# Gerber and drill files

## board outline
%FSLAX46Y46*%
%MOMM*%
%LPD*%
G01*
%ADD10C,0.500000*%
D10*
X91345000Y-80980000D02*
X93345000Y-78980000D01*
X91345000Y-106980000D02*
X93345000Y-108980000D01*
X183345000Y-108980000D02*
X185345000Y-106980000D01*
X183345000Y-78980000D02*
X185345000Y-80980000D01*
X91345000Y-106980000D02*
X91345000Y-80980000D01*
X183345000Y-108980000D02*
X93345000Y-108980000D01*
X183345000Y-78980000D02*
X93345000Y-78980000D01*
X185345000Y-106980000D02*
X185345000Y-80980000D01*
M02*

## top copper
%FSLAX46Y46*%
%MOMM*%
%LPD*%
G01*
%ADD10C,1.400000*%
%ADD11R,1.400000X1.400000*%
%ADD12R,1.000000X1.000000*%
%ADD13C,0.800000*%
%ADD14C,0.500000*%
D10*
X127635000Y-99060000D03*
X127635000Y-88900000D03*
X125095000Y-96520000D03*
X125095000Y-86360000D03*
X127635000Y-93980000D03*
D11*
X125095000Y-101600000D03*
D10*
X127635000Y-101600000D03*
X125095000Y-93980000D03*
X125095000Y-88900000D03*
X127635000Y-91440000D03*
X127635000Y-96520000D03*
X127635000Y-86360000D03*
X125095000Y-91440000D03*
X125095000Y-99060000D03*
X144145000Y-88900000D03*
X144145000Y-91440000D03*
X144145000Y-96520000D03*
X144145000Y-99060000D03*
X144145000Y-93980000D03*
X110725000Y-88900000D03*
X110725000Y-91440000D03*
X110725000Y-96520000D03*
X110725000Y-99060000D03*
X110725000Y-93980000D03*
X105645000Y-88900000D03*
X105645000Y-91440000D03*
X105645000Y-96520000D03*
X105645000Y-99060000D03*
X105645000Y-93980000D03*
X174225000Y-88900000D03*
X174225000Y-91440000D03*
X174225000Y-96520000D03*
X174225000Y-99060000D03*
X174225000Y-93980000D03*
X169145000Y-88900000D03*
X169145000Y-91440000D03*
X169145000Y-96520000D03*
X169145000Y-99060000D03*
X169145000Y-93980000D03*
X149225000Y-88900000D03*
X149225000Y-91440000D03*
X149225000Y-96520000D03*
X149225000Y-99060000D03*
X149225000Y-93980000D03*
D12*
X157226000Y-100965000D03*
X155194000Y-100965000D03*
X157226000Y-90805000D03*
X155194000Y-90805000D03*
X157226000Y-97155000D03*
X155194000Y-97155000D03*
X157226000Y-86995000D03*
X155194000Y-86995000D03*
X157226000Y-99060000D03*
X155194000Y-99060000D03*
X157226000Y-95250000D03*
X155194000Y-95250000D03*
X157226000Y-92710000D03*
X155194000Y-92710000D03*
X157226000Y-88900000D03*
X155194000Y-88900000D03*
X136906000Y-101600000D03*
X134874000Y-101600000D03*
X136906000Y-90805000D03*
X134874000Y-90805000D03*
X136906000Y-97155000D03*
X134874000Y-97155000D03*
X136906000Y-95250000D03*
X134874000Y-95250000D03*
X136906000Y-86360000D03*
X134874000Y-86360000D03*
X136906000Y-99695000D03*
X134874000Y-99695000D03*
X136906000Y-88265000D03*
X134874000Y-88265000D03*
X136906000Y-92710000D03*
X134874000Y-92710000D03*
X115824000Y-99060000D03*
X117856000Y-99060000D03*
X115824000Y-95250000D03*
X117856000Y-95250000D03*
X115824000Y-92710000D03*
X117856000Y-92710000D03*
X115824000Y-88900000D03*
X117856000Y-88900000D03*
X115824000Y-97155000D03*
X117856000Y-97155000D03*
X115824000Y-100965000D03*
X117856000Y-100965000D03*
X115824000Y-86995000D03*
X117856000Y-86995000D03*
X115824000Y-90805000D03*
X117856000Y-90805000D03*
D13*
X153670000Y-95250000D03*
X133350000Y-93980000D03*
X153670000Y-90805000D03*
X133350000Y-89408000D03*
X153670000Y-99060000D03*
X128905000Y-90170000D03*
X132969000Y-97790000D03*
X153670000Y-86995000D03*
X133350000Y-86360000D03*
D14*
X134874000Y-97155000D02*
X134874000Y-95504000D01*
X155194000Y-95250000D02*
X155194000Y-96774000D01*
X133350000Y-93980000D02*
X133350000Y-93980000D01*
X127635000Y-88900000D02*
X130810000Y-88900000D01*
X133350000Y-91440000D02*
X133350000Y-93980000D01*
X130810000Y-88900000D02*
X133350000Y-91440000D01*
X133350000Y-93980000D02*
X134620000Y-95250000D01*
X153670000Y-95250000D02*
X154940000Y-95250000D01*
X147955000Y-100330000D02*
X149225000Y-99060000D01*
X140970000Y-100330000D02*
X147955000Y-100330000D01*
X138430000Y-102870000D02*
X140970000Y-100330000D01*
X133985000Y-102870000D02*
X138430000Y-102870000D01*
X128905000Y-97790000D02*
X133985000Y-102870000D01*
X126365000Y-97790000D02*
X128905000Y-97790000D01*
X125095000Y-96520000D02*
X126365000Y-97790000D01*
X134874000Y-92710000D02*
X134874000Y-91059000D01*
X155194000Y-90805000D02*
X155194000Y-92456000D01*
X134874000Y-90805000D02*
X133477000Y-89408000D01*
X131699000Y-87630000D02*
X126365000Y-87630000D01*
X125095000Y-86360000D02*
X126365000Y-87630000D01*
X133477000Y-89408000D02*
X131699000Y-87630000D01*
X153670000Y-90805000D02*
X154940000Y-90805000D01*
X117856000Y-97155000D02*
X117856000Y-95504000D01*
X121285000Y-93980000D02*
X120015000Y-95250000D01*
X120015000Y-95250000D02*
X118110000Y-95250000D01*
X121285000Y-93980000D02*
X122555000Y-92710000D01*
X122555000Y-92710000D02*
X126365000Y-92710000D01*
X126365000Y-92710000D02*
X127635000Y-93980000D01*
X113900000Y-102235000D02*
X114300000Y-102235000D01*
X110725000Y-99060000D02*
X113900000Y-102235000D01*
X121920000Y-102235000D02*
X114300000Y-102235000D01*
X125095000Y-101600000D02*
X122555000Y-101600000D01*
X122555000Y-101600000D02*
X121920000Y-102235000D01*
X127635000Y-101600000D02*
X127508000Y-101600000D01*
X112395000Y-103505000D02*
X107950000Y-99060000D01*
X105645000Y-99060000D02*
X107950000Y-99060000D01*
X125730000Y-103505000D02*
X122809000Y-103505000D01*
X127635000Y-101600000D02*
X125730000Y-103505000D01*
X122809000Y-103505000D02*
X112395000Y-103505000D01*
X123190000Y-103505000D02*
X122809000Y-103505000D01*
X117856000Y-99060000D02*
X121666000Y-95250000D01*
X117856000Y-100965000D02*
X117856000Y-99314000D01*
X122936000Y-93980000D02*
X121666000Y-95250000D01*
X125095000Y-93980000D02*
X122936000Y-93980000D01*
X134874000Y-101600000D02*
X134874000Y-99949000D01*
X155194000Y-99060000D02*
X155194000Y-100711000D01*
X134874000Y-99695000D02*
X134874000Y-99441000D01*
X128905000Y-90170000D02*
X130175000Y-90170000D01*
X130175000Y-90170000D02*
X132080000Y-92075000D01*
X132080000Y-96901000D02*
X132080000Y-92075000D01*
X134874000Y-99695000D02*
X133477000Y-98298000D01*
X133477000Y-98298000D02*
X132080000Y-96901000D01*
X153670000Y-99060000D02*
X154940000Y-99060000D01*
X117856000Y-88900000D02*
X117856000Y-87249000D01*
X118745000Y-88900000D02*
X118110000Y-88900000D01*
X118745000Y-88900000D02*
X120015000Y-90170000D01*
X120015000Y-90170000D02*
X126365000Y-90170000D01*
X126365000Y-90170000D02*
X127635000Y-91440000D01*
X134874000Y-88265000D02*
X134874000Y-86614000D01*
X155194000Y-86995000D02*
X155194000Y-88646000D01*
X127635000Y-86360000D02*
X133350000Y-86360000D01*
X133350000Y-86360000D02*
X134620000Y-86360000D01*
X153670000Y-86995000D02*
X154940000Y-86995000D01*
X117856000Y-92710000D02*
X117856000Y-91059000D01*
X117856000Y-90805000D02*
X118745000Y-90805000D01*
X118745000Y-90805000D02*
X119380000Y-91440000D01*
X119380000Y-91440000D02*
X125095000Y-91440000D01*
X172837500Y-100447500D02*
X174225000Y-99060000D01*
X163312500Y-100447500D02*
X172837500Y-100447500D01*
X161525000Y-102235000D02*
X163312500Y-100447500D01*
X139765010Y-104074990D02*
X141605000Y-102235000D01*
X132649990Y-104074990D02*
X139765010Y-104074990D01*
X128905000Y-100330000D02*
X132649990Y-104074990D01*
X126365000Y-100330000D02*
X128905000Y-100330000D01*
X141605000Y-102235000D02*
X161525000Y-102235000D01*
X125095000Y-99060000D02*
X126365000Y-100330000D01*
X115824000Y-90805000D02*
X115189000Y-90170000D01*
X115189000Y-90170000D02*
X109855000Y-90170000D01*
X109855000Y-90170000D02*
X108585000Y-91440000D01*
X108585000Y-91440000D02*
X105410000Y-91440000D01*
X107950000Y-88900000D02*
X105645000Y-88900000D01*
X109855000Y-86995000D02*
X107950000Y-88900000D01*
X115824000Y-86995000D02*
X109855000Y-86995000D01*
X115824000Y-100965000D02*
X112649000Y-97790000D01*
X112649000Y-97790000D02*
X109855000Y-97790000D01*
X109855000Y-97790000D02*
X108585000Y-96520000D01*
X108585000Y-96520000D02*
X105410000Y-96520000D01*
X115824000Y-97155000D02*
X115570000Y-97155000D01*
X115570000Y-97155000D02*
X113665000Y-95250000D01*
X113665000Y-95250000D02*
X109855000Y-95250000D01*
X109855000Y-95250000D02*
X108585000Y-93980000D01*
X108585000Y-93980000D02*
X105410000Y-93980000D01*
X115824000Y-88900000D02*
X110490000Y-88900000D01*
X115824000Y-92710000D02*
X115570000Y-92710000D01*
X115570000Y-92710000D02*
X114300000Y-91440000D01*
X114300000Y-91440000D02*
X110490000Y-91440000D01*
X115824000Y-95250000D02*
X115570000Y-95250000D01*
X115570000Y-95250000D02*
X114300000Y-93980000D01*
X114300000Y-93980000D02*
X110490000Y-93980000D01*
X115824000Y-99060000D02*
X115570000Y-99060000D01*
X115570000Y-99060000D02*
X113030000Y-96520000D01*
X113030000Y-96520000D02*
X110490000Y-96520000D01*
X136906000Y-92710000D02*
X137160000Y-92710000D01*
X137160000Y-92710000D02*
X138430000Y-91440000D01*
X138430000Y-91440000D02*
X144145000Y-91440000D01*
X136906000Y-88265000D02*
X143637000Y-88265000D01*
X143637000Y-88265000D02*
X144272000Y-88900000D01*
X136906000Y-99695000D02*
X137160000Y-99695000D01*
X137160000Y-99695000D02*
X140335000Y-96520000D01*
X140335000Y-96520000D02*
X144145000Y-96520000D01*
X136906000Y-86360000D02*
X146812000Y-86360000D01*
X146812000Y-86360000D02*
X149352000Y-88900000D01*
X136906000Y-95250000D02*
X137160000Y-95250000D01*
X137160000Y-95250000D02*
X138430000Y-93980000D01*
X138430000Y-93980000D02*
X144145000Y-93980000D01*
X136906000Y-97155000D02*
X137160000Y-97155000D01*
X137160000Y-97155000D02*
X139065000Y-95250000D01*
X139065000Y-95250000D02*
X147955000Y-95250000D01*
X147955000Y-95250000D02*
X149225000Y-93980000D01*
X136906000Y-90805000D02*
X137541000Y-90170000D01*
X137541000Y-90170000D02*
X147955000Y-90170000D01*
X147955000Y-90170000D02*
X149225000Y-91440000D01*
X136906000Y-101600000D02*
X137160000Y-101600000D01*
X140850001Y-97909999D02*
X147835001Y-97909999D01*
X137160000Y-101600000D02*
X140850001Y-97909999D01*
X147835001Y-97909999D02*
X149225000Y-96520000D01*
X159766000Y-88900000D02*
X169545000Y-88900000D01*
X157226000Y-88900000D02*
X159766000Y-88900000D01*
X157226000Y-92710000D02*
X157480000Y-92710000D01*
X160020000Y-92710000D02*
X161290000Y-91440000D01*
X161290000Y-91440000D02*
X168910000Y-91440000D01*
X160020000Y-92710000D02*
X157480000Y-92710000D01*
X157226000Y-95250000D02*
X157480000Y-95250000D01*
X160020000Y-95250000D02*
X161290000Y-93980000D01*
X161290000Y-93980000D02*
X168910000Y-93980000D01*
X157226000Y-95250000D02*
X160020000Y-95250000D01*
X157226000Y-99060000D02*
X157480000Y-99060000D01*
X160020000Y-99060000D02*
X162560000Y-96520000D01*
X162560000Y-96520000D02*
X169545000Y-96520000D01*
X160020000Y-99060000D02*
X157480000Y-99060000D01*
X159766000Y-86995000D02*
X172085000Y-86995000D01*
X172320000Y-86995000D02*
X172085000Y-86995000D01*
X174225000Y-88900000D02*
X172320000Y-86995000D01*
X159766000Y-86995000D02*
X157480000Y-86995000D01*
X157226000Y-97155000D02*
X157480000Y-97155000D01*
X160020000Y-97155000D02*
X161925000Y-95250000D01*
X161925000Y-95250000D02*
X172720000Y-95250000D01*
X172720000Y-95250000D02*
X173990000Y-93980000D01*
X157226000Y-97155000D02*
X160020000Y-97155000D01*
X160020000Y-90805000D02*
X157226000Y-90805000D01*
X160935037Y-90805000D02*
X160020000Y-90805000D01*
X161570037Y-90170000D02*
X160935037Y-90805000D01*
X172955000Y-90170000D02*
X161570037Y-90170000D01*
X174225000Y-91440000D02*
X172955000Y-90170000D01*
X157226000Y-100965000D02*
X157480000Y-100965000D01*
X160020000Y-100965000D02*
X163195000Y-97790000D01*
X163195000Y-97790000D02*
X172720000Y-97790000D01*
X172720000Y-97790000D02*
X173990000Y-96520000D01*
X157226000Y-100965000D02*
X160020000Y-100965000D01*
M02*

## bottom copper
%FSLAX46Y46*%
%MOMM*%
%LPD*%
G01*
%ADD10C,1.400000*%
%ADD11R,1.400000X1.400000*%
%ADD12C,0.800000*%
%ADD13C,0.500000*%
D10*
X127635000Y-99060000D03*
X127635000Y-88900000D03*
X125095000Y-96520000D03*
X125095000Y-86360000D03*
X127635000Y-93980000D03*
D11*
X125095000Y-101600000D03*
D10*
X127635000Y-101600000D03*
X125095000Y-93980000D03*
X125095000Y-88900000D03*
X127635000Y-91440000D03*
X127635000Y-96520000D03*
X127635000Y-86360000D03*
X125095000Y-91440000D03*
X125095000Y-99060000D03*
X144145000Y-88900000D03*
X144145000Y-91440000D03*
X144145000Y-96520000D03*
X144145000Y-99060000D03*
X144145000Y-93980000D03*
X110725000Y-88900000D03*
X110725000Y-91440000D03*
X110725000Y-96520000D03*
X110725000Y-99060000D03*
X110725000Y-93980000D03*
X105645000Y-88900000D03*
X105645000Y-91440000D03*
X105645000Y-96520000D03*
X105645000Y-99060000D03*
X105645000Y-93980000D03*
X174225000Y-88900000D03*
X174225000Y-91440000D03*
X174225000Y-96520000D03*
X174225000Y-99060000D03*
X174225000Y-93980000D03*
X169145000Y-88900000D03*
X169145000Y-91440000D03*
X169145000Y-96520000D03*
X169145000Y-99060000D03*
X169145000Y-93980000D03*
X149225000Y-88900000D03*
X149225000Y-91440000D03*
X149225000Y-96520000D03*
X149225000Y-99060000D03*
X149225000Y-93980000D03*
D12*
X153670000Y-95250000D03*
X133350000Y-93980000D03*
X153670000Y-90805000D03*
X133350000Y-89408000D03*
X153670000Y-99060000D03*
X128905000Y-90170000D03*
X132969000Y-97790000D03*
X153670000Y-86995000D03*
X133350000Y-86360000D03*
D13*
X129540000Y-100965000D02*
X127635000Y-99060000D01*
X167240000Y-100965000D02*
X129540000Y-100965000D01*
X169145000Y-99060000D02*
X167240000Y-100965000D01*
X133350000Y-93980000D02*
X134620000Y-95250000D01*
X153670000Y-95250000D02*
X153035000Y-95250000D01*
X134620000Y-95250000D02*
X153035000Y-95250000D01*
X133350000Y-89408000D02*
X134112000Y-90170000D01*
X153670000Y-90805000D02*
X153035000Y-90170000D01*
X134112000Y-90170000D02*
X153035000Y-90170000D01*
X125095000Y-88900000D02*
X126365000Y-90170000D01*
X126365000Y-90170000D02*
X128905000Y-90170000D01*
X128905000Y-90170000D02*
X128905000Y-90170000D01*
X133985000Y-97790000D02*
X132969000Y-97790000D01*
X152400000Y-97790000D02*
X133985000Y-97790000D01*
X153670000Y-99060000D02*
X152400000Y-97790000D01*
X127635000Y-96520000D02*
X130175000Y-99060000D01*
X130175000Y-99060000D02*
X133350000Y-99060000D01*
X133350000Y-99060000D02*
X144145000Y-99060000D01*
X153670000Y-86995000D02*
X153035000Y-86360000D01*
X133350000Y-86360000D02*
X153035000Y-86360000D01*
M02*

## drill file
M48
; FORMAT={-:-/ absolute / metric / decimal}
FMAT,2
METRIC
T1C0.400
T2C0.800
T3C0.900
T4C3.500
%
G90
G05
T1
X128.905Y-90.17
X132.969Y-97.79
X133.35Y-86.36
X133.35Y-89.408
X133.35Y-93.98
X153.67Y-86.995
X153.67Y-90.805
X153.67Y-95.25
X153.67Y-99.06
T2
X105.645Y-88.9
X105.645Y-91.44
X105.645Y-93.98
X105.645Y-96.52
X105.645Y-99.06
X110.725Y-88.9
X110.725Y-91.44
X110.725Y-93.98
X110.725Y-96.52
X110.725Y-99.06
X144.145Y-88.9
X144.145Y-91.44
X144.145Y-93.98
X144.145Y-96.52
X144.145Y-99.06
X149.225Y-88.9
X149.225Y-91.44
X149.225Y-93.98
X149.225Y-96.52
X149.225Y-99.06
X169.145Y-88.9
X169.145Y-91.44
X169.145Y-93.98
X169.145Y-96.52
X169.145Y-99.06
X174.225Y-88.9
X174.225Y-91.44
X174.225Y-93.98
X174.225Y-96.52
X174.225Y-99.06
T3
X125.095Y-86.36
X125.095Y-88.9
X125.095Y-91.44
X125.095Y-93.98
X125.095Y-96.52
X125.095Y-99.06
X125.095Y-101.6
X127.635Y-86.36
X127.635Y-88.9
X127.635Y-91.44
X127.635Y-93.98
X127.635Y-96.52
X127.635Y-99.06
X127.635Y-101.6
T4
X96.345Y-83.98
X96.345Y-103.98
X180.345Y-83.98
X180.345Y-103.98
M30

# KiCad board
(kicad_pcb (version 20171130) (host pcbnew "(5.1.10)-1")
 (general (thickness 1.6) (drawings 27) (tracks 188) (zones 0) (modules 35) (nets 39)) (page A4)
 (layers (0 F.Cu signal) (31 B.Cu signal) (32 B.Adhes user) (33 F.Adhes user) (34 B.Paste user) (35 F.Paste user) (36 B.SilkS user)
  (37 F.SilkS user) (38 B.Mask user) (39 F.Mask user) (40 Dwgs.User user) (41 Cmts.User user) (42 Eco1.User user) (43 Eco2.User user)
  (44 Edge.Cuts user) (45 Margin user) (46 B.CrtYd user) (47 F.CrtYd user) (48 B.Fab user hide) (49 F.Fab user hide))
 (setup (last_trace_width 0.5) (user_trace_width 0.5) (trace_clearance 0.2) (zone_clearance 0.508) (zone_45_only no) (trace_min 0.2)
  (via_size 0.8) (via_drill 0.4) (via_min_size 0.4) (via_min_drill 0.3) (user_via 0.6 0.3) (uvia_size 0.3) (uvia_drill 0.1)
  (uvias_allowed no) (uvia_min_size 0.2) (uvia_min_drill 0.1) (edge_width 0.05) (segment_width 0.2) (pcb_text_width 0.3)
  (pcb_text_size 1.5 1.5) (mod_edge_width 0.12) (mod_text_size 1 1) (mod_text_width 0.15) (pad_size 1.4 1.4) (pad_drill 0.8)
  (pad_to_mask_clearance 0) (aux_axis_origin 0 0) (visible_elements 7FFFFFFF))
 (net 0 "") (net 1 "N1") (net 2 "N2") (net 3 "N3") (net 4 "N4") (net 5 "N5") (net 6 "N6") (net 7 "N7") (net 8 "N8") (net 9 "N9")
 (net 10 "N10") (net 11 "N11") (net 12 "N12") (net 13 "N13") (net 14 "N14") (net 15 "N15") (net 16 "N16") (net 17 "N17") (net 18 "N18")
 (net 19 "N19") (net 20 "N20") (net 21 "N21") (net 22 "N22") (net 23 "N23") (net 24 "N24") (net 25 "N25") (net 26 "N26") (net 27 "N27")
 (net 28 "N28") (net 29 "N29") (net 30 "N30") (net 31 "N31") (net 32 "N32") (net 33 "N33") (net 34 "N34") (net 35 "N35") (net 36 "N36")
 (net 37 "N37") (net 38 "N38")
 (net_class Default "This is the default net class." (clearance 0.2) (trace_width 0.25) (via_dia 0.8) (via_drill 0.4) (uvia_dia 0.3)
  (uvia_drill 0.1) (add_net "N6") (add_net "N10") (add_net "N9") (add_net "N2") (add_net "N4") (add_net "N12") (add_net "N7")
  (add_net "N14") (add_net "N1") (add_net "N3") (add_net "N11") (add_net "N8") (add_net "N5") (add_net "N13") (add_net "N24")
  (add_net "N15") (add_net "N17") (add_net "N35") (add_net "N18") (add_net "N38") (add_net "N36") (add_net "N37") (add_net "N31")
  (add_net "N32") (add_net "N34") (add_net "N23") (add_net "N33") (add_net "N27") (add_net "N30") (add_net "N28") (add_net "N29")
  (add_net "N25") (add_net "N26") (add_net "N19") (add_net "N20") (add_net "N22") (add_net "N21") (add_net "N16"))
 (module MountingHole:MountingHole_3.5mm (layer F.Cu) (at 96.345 103.98)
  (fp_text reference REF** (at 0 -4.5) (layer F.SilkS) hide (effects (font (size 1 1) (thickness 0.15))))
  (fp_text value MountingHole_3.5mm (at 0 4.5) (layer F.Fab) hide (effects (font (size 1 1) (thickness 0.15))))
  (pad 1 np_thru_hole circle (at 0 0) (size 3.5 3.5) (drill 3.5) (layers *.Cu *.Mask)))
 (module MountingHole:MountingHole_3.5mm (layer F.Cu) (at 96.345 83.98)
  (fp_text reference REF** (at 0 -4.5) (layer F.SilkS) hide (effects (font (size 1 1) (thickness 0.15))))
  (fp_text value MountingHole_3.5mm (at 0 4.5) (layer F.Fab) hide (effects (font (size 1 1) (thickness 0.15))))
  (pad 1 np_thru_hole circle (at 0 0) (size 3.5 3.5) (drill 3.5) (layers *.Cu *.Mask)))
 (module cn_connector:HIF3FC (layer B.Cu) (at 126.365 93.98)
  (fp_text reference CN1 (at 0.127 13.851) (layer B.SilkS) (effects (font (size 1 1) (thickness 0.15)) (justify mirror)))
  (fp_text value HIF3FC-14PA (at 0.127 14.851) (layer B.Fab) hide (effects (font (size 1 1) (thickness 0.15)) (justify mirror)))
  (pad 4 thru_hole circle (at 1.27 5.08) (size 1.4 1.4) (drill 0.9) (layers *.Cu *.Mask) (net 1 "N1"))
  (pad 12 thru_hole circle (at 1.27 -5.08) (size 1.4 1.4) (drill 0.9) (layers *.Cu *.Mask) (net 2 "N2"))
  (pad 5 thru_hole circle (at -1.27 2.54) (size 1.4 1.4) (drill 0.9) (layers *.Cu *.Mask) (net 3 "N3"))
  (pad 13 thru_hole circle (at -1.27 -7.62) (size 1.4 1.4) (drill 0.9) (layers *.Cu *.Mask) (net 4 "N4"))
  (pad 8 thru_hole circle (at 1.27 0) (size 1.4 1.4) (drill 0.9) (layers *.Cu *.Mask) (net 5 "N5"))
  (pad 1 thru_hole rect (at -1.27 7.62) (size 1.4 1.4) (drill 0.9) (layers *.Cu *.Mask) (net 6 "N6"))
  (pad 2 thru_hole circle (at 1.27 7.62) (size 1.4 1.4) (drill 0.9) (layers *.Cu *.Mask) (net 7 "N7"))
  (pad 7 thru_hole circle (at -1.27 0) (size 1.4 1.4) (drill 0.9) (layers *.Cu *.Mask) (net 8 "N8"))
  (pad 11 thru_hole circle (at -1.27 -5.08) (size 1.4 1.4) (drill 0.9) (layers *.Cu *.Mask) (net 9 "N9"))
  (pad 10 thru_hole circle (at 1.27 -2.54) (size 1.4 1.4) (drill 0.9) (layers *.Cu *.Mask) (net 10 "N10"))
  (pad 6 thru_hole circle (at 1.27 2.54) (size 1.4 1.4) (drill 0.9) (layers *.Cu *.Mask) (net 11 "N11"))
  (pad 14 thru_hole circle (at 1.27 -7.62) (size 1.4 1.4) (drill 0.9) (layers *.Cu *.Mask) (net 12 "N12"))
  (pad 9 thru_hole circle (at -1.27 -2.54) (size 1.4 1.4) (drill 0.9) (layers *.Cu *.Mask) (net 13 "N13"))
  (pad 3 thru_hole circle (at -1.27 5.08) (size 1.4 1.4) (drill 0.9) (layers *.Cu *.Mask) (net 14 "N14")))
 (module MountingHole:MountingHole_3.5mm (layer F.Cu) (at 180.345 103.98)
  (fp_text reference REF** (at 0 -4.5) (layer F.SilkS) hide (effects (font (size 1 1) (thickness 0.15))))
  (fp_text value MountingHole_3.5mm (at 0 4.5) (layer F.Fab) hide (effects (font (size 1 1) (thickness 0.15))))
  (pad 1 np_thru_hole circle (at 0 0) (size 3.5 3.5) (drill 3.5) (layers *.Cu *.Mask)))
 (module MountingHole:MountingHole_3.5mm (layer F.Cu) (at 180.345 83.98)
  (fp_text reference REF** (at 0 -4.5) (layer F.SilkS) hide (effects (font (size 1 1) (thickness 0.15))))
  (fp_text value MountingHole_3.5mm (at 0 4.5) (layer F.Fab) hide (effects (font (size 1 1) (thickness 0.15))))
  (pad 1 np_thru_hole circle (at 0 0) (size 3.5 3.5) (drill 3.5) (layers *.Cu *.Mask)))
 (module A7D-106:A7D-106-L (layer F.Cu) (at 144.145 88.9)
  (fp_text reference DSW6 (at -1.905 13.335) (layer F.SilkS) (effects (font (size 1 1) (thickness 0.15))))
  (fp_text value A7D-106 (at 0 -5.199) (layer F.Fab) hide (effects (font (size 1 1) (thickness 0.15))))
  (pad 8 thru_hole circle (at 0 0) (size 1.4 1.4) (drill 0.8) (layers *.Cu *.Mask) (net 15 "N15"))
  (pad 4 thru_hole circle (at 0 2.54) (size 1.4 1.4) (drill 0.8) (layers *.Cu *.Mask) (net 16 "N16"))
  (pad 1 thru_hole circle (at 0 7.62) (size 1.4 1.4) (drill 0.8) (layers *.Cu *.Mask) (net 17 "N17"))
  (pad C thru_hole circle (at 0 10.16) (size 1.4 1.4) (drill 0.8) (layers *.Cu *.Mask) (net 11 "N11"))
  (pad 2 thru_hole circle (at 0 5.08) (size 1.4 1.4) (drill 0.8) (layers *.Cu *.Mask) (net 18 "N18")))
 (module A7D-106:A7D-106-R (layer F.Cu) (at 110.725 88.9)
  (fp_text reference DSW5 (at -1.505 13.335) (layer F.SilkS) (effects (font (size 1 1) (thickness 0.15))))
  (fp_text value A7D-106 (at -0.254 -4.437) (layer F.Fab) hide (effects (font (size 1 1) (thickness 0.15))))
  (pad 8 thru_hole circle (at 0 0) (size 1.4 1.4) (drill 0.8) (layers *.Cu *.Mask) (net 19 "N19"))
  (pad 4 thru_hole circle (at 0 2.54) (size 1.4 1.4) (drill 0.8) (layers *.Cu *.Mask) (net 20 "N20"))
  (pad 1 thru_hole circle (at 0 7.62) (size 1.4 1.4) (drill 0.8) (layers *.Cu *.Mask) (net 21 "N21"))
  (pad C thru_hole circle (at 0 10.16) (size 1.4 1.4) (drill 0.8) (layers *.Cu *.Mask) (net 6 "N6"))
  (pad 2 thru_hole circle (at 0 5.08) (size 1.4 1.4) (drill 0.8) (layers *.Cu *.Mask) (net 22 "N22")))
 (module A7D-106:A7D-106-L (layer F.Cu) (at 105.645 88.9)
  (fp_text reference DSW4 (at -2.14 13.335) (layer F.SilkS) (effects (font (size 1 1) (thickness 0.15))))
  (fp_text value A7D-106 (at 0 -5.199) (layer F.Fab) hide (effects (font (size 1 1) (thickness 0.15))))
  (pad 8 thru_hole circle (at 0 0) (size 1.4 1.4) (drill 0.8) (layers *.Cu *.Mask) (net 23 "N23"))
  (pad 4 thru_hole circle (at 0 2.54) (size 1.4 1.4) (drill 0.8) (layers *.Cu *.Mask) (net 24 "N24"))
  (pad 1 thru_hole circle (at 0 7.62) (size 1.4 1.4) (drill 0.8) (layers *.Cu *.Mask) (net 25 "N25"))
  (pad C thru_hole circle (at 0 10.16) (size 1.4 1.4) (drill 0.8) (layers *.Cu *.Mask) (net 7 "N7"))
  (pad 2 thru_hole circle (at 0 5.08) (size 1.4 1.4) (drill 0.8) (layers *.Cu *.Mask) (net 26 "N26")))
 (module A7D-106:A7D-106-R (layer F.Cu) (at 174.225 88.9)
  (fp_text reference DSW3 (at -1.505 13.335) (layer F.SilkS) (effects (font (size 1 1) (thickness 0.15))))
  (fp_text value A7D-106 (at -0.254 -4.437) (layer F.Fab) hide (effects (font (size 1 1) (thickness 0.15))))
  (pad 8 thru_hole circle (at 0 0) (size 1.4 1.4) (drill 0.8) (layers *.Cu *.Mask) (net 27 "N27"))
  (pad 4 thru_hole circle (at 0 2.54) (size 1.4 1.4) (drill 0.8) (layers *.Cu *.Mask) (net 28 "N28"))
  (pad 1 thru_hole circle (at 0 7.62) (size 1.4 1.4) (drill 0.8) (layers *.Cu *.Mask) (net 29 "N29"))
  (pad C thru_hole circle (at 0 10.16) (size 1.4 1.4) (drill 0.8) (layers *.Cu *.Mask) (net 14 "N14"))
  (pad 2 thru_hole circle (at 0 5.08) (size 1.4 1.4) (drill 0.8) (layers *.Cu *.Mask) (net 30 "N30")))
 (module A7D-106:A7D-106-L (layer F.Cu) (at 169.145 88.9)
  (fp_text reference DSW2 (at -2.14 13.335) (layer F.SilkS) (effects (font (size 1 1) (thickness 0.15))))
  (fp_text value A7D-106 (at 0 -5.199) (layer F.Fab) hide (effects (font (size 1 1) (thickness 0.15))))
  (pad 8 thru_hole circle (at 0 0) (size 1.4 1.4) (drill 0.8) (layers *.Cu *.Mask) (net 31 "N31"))
  (pad 4 thru_hole circle (at 0 2.54) (size 1.4 1.4) (drill 0.8) (layers *.Cu *.Mask) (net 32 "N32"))
  (pad 1 thru_hole circle (at 0 7.62) (size 1.4 1.4) (drill 0.8) (layers *.Cu *.Mask) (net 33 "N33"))
  (pad C thru_hole circle (at 0 10.16) (size 1.4 1.4) (drill 0.8) (layers *.Cu *.Mask) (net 1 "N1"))
  (pad 2 thru_hole circle (at 0 5.08) (size 1.4 1.4) (drill 0.8) (layers *.Cu *.Mask) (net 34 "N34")))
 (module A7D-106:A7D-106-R (layer F.Cu) (at 149.225 88.9)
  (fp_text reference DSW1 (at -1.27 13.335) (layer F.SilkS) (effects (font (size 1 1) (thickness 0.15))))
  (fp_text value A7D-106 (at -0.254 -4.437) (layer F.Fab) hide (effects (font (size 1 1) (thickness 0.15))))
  (pad 8 thru_hole circle (at 0 0) (size 1.4 1.4) (drill 0.8) (layers *.Cu *.Mask) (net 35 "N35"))
  (pad 4 thru_hole circle (at 0 2.54) (size 1.4 1.4) (drill 0.8) (layers *.Cu *.Mask) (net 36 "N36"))
  (pad 1 thru_hole circle (at 0 7.62) (size 1.4 1.4) (drill 0.8) (layers *.Cu *.Mask) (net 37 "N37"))
  (pad C thru_hole circle (at 0 10.16) (size 1.4 1.4) (drill 0.8) (layers *.Cu *.Mask) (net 3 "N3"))
  (pad 2 thru_hole circle (at 0 5.08) (size 1.4 1.4) (drill 0.8) (layers *.Cu *.Mask) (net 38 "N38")))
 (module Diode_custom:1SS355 (layer F.Cu) (at 156.21 100.965)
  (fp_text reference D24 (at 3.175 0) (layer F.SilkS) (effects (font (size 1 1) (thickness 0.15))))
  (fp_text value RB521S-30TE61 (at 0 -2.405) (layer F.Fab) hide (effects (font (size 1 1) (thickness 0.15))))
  (pad 2 smd rect (at 1.016 0) (size 1 1) (layers F.Cu F.Paste F.Mask) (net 29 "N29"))
  (pad 1 smd rect (at -1.016 0) (size 1 1) (layers F.Cu F.Paste F.Mask) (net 9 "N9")))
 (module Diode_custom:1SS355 (layer F.Cu) (at 156.21 90.805)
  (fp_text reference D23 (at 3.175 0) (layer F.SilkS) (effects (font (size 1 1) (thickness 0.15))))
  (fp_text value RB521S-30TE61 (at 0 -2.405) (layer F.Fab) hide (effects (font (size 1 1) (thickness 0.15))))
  (pad 2 smd rect (at 1.016 0) (size 1 1) (layers F.Cu F.Paste F.Mask) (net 28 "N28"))
  (pad 1 smd rect (at -1.016 0) (size 1 1) (layers F.Cu F.Paste F.Mask) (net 4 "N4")))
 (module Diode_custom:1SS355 (layer F.Cu) (at 156.21 97.155)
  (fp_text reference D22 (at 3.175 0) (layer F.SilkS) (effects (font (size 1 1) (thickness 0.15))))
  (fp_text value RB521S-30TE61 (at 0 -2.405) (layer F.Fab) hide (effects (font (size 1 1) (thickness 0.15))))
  (pad 2 smd rect (at 1.016 0) (size 1 1) (layers F.Cu F.Paste F.Mask) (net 30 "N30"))
  (pad 1 smd rect (at -1.016 0) (size 1 1) (layers F.Cu F.Paste F.Mask) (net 2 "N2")))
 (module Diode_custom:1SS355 (layer F.Cu) (at 156.21 86.995)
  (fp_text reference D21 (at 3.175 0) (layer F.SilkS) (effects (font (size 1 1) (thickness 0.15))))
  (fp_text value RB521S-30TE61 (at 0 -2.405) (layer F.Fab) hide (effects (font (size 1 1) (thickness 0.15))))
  (pad 2 smd rect (at 1.016 0) (size 1 1) (layers F.Cu F.Paste F.Mask) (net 27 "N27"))
  (pad 1 smd rect (at -1.016 0) (size 1 1) (layers F.Cu F.Paste F.Mask) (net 12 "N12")))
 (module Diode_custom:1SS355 (layer F.Cu) (at 156.21 99.06)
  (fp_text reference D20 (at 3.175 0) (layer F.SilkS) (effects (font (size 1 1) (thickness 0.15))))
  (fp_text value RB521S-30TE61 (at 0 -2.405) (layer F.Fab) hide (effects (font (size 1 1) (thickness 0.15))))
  (pad 2 smd rect (at 1.016 0) (size 1 1) (layers F.Cu F.Paste F.Mask) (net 33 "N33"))
  (pad 1 smd rect (at -1.016 0) (size 1 1) (layers F.Cu F.Paste F.Mask) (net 9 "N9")))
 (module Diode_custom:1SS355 (layer F.Cu) (at 156.21 95.25)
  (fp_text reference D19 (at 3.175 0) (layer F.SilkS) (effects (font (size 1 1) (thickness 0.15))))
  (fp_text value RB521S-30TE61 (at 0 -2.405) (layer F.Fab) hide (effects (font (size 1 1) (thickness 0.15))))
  (pad 2 smd rect (at 1.016 0) (size 1 1) (layers F.Cu F.Paste F.Mask) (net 34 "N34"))
  (pad 1 smd rect (at -1.016 0) (size 1 1) (layers F.Cu F.Paste F.Mask) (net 2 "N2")))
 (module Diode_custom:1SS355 (layer F.Cu) (at 156.21 92.71)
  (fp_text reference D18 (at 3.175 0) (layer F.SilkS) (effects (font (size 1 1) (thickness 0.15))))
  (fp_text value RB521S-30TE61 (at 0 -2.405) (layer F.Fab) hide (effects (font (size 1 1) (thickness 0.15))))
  (pad 2 smd rect (at 1.016 0) (size 1 1) (layers F.Cu F.Paste F.Mask) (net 32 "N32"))
  (pad 1 smd rect (at -1.016 0) (size 1 1) (layers F.Cu F.Paste F.Mask) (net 4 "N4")))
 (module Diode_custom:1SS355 (layer F.Cu) (at 156.21 88.9)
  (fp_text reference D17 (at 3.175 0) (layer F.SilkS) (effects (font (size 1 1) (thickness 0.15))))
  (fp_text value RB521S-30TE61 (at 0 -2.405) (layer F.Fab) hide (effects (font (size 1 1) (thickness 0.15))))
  (pad 2 smd rect (at 1.016 0) (size 1 1) (layers F.Cu F.Paste F.Mask) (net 31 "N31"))
  (pad 1 smd rect (at -1.016 0) (size 1 1) (layers F.Cu F.Paste F.Mask) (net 12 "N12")))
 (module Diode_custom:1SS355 (layer F.Cu) (at 135.89 101.6)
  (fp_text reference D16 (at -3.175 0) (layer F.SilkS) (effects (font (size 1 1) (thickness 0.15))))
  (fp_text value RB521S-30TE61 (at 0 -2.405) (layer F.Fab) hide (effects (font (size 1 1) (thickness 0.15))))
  (pad 2 smd rect (at 1.016 0) (size 1 1) (layers F.Cu F.Paste F.Mask) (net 37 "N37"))
  (pad 1 smd rect (at -1.016 0) (size 1 1) (layers F.Cu F.Paste F.Mask) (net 9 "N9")))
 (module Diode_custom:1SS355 (layer F.Cu) (at 135.89 90.805)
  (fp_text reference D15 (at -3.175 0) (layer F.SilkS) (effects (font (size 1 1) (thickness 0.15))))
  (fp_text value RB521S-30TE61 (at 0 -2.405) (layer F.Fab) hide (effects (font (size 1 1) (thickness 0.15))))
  (pad 2 smd rect (at 1.016 0) (size 1 1) (layers F.Cu F.Paste F.Mask) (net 36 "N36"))
  (pad 1 smd rect (at -1.016 0) (size 1 1) (layers F.Cu F.Paste F.Mask) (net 4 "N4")))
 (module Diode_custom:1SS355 (layer F.Cu) (at 135.89 97.155)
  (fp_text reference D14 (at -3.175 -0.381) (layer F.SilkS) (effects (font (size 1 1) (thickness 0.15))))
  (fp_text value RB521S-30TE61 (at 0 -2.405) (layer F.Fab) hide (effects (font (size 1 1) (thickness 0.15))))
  (pad 2 smd rect (at 1.016 0) (size 1 1) (layers F.Cu F.Paste F.Mask) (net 38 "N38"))
  (pad 1 smd rect (at -1.016 0) (size 1 1) (layers F.Cu F.Paste F.Mask) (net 2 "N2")))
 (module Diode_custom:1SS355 (layer F.Cu) (at 135.89 95.25)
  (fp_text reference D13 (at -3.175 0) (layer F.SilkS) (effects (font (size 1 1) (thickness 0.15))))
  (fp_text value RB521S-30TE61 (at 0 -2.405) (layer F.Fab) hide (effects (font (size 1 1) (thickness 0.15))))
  (pad 2 smd rect (at 1.016 0) (size 1 1) (layers F.Cu F.Paste F.Mask) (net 18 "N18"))
  (pad 1 smd rect (at -1.016 0) (size 1 1) (layers F.Cu F.Paste F.Mask) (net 2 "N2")))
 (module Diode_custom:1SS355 (layer F.Cu) (at 135.89 86.36)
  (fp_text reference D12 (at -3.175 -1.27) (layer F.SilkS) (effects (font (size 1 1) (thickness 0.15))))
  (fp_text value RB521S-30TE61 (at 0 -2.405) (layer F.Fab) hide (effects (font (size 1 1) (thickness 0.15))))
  (pad 2 smd rect (at 1.016 0) (size 1 1) (layers F.Cu F.Paste F.Mask) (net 35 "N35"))
  (pad 1 smd rect (at -1.016 0) (size 1 1) (layers F.Cu F.Paste F.Mask) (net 12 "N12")))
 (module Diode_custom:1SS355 (layer F.Cu) (at 135.89 99.695)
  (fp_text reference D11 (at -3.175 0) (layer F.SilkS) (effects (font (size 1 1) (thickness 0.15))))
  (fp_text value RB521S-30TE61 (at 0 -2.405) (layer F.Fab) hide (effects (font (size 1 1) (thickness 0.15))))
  (pad 2 smd rect (at 1.016 0) (size 1 1) (layers F.Cu F.Paste F.Mask) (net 17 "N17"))
  (pad 1 smd rect (at -1.016 0) (size 1 1) (layers F.Cu F.Paste F.Mask) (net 9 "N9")))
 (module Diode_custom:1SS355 (layer F.Cu) (at 135.89 88.265)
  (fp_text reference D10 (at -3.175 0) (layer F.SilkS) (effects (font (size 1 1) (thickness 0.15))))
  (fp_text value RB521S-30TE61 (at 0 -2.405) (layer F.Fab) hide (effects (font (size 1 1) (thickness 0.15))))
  (pad 2 smd rect (at 1.016 0) (size 1 1) (layers F.Cu F.Paste F.Mask) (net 15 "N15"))
  (pad 1 smd rect (at -1.016 0) (size 1 1) (layers F.Cu F.Paste F.Mask) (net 12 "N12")))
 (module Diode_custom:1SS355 (layer F.Cu) (at 135.89 92.71)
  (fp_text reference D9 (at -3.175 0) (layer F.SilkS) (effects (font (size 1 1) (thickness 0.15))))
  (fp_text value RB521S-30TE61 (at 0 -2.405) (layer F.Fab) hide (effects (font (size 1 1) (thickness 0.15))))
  (pad 2 smd rect (at 1.016 0) (size 1 1) (layers F.Cu F.Paste F.Mask) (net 16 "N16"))
  (pad 1 smd rect (at -1.016 0) (size 1 1) (layers F.Cu F.Paste F.Mask) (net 4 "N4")))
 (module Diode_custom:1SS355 (layer F.Cu) (at 116.84 99.06 180)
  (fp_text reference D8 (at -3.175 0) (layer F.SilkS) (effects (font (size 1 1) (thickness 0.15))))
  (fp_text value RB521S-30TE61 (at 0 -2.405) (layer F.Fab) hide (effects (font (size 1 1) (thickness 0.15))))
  (pad 2 smd rect (at 1.016 0 180) (size 1 1) (layers F.Cu F.Paste F.Mask) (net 21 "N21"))
  (pad 1 smd rect (at -1.016 0 180) (size 1 1) (layers F.Cu F.Paste F.Mask) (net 8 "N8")))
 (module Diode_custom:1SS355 (layer F.Cu) (at 116.84 95.25 180)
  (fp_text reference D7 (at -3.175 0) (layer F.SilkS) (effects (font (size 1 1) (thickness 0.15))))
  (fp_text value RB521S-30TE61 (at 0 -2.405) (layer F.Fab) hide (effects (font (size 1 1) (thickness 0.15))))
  (pad 2 smd rect (at 1.016 0 180) (size 1 1) (layers F.Cu F.Paste F.Mask) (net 22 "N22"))
  (pad 1 smd rect (at -1.016 0 180) (size 1 1) (layers F.Cu F.Paste F.Mask) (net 5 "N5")))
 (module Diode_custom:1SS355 (layer F.Cu) (at 116.84 92.71 180)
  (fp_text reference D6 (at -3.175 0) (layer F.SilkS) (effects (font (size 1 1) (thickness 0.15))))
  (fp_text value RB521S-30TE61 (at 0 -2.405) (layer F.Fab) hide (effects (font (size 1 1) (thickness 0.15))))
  (pad 2 smd rect (at 1.016 0 180) (size 1 1) (layers F.Cu F.Paste F.Mask) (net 20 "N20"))
  (pad 1 smd rect (at -1.016 0 180) (size 1 1) (layers F.Cu F.Paste F.Mask) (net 13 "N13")))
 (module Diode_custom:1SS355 (layer F.Cu) (at 116.84 88.9 180)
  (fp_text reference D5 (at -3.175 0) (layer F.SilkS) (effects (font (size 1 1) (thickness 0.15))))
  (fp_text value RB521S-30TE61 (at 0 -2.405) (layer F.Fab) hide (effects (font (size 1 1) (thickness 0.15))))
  (pad 2 smd rect (at 1.016 0 180) (size 1 1) (layers F.Cu F.Paste F.Mask) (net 19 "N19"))
  (pad 1 smd rect (at -1.016 0 180) (size 1 1) (layers F.Cu F.Paste F.Mask) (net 10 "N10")))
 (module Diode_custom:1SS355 (layer F.Cu) (at 116.84 97.155 180)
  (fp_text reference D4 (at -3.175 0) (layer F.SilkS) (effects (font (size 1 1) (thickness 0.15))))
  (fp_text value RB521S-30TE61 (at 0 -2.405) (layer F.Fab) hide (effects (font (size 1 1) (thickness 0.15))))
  (pad 2 smd rect (at 1.016 0 180) (size 1 1) (layers F.Cu F.Paste F.Mask) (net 26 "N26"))
  (pad 1 smd rect (at -1.016 0 180) (size 1 1) (layers F.Cu F.Paste F.Mask) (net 5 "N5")))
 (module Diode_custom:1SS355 (layer F.Cu) (at 116.84 100.965 180)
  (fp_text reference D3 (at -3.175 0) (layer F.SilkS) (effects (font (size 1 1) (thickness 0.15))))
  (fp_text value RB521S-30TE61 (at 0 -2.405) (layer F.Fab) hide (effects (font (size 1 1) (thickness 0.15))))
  (pad 2 smd rect (at 1.016 0 180) (size 1 1) (layers F.Cu F.Paste F.Mask) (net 25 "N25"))
  (pad 1 smd rect (at -1.016 0 180) (size 1 1) (layers F.Cu F.Paste F.Mask) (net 8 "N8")))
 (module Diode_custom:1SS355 (layer F.Cu) (at 116.84 86.995 180)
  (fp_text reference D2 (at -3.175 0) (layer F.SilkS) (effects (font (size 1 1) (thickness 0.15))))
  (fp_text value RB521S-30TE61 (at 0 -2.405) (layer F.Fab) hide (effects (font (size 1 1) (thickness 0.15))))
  (pad 2 smd rect (at 1.016 0 180) (size 1 1) (layers F.Cu F.Paste F.Mask) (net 23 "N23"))
  (pad 1 smd rect (at -1.016 0 180) (size 1 1) (layers F.Cu F.Paste F.Mask) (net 10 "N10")))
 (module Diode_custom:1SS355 (layer F.Cu) (at 116.84 90.805 180)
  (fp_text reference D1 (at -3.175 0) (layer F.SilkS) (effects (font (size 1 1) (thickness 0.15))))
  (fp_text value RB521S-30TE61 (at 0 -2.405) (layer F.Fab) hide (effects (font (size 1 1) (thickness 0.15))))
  (pad 2 smd rect (at 1.016 0 180) (size 1 1) (layers F.Cu F.Paste F.Mask) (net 24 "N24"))
  (pad 1 smd rect (at -1.016 0 180) (size 1 1) (layers F.Cu F.Paste F.Mask) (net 13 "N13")))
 (gr_line (start 91.345 80.98) (end 93.345 78.98) (layer Edge.Cuts) (width 0.5))
 (gr_line (start 91.345 106.98) (end 93.345 108.98) (layer Edge.Cuts) (width 0.5))
 (gr_line (start 183.345 108.98) (end 185.345 106.98) (layer Edge.Cuts) (width 0.5))
 (gr_line (start 183.345 78.98) (end 185.345 80.98) (layer Edge.Cuts) (width 0.5))
 (gr_line (start 91.345 106.98) (end 91.345 80.98) (layer Edge.Cuts) (width 0.5))
 (gr_line (start 183.345 108.98) (end 93.345 108.98) (layer Edge.Cuts) (width 0.5))
 (gr_line (start 183.345 78.98) (end 93.345 78.98) (layer Edge.Cuts) (width 0.5))
 (gr_line (start 185.345 106.98) (end 185.345 80.98) (layer Edge.Cuts) (width 0.5))
 (segment (start 129.54 100.965) (end 127.635 99.06) (width 0.5) (layer B.Cu) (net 1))
 (segment (start 167.24 100.965) (end 129.54 100.965) (width 0.5) (layer B.Cu) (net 1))
 (segment (start 169.145 99.06) (end 167.24 100.965) (width 0.5) (layer B.Cu) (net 1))
 (via (at 153.67 95.25) (size 0.8) (drill 0.4) (layers F.Cu B.Cu) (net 2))
 (segment (start 134.874 97.155) (end 134.874 95.504) (width 0.5) (layer F.Cu) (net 2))
 (segment (start 155.194 95.25) (end 155.194 96.774) (width 0.5) (layer F.Cu) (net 2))
 (segment (start 133.35 93.98) (end 133.35 93.98) (width 0.5) (layer F.Cu) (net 2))
 (segment (start 127.635 88.9) (end 130.81 88.9) (width 0.5) (layer F.Cu) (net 2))
 (segment (start 133.35 91.44) (end 133.35 93.98) (width 0.5) (layer F.Cu) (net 2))
 (segment (start 130.81 88.9) (end 133.35 91.44) (width 0.5) (layer F.Cu) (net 2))
 (segment (start 133.35 93.98) (end 134.62 95.25) (width 0.5) (layer F.Cu) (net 2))
 (via (at 133.35 93.98) (size 0.8) (drill 0.4) (layers F.Cu B.Cu) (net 2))
 (segment (start 133.35 93.98) (end 134.62 95.25) (width 0.5) (layer B.Cu) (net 2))
 (segment (start 153.67 95.25) (end 153.035 95.25) (width 0.5) (layer B.Cu) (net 2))
 (segment (start 134.62 95.25) (end 153.035 95.25) (width 0.5) (layer B.Cu) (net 2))
 (segment (start 153.67 95.25) (end 154.94 95.25) (width 0.5) (layer F.Cu) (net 2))
 (segment (start 147.955 100.33) (end 149.225 99.06) (width 0.5) (layer F.Cu) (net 3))
 (segment (start 140.97 100.33) (end 147.955 100.33) (width 0.5) (layer F.Cu) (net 3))
 (segment (start 138.43 102.87) (end 140.97 100.33) (width 0.5) (layer F.Cu) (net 3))
 (segment (start 133.985 102.87) (end 138.43 102.87) (width 0.5) (layer F.Cu) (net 3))
 (segment (start 128.905 97.79) (end 133.985 102.87) (width 0.5) (layer F.Cu) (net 3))
 (segment (start 126.365 97.79) (end 128.905 97.79) (width 0.5) (layer F.Cu) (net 3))
 (segment (start 125.095 96.52) (end 126.365 97.79) (width 0.5) (layer F.Cu) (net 3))
 (via (at 153.67 90.805) (size 0.8) (drill 0.4) (layers F.Cu B.Cu) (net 4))
 (segment (start 134.874 92.71) (end 134.874 91.059) (width 0.5) (layer F.Cu) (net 4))
 (segment (start 155.194 90.805) (end 155.194 92.456) (width 0.5) (layer F.Cu) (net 4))
 (segment (start 134.874 90.805) (end 133.477 89.408) (width 0.5) (layer F.Cu) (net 4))
 (segment (start 131.699 87.63) (end 126.365 87.63) (width 0.5) (layer F.Cu) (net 4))
 (segment (start 125.095 86.36) (end 126.365 87.63) (width 0.5) (layer F.Cu) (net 4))
 (segment (start 133.477 89.408) (end 131.699 87.63) (width 0.5) (layer F.Cu) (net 4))
 (via (at 133.35 89.408) (size 0.8) (drill 0.4) (layers F.Cu B.Cu) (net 4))
 (segment (start 133.35 89.408) (end 134.112 90.17) (width 0.5) (layer B.Cu) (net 4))
 (segment (start 153.67 90.805) (end 153.035 90.17) (width 0.5) (layer B.Cu) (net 4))
 (segment (start 134.112 90.17) (end 153.035 90.17) (width 0.5) (layer B.Cu) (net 4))
 (segment (start 153.67 90.805) (end 154.94 90.805) (width 0.5) (layer F.Cu) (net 4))
 (segment (start 117.856 97.155) (end 117.856 95.504) (width 0.5) (layer F.Cu) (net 5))
 (segment (start 121.285 93.98) (end 120.015 95.25) (width 0.5) (layer F.Cu) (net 5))
 (segment (start 120.015 95.25) (end 118.11 95.25) (width 0.5) (layer F.Cu) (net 5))
 (segment (start 121.285 93.98) (end 122.555 92.71) (width 0.5) (layer F.Cu) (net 5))
 (segment (start 122.555 92.71) (end 126.365 92.71) (width 0.5) (layer F.Cu) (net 5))
 (segment (start 126.365 92.71) (end 127.635 93.98) (width 0.5) (layer F.Cu) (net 5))
 (segment (start 113.9 102.235) (end 114.3 102.235) (width 0.5) (layer F.Cu) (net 6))
 (segment (start 110.725 99.06) (end 113.9 102.235) (width 0.5) (layer F.Cu) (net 6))
 (segment (start 121.92 102.235) (end 114.3 102.235) (width 0.5) (layer F.Cu) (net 6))
 (segment (start 125.095 101.6) (end 122.555 101.6) (width 0.5) (layer F.Cu) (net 6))
 (segment (start 122.555 101.6) (end 121.92 102.235) (width 0.5) (layer F.Cu) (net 6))
 (segment (start 127.635 101.6) (end 127.508 101.6) (width 0.5) (layer F.Cu) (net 7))
 (segment (start 112.395 103.505) (end 107.95 99.06) (width 0.5) (layer F.Cu) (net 7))
 (segment (start 105.645 99.06) (end 107.95 99.06) (width 0.5) (layer F.Cu) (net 7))
 (segment (start 125.73 103.505) (end 122.809 103.505) (width 0.5) (layer F.Cu) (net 7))
 (segment (start 127.635 101.6) (end 125.73 103.505) (width 0.5) (layer F.Cu) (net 7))
 (segment (start 122.809 103.505) (end 112.395 103.505) (width 0.5) (layer F.Cu) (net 7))
 (segment (start 123.19 103.505) (end 122.809 103.505) (width 0.5) (layer F.Cu) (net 7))
 (segment (start 117.856 99.06) (end 121.666 95.25) (width 0.5) (layer F.Cu) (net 8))
 (segment (start 117.856 100.965) (end 117.856 99.314) (width 0.5) (layer F.Cu) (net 8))
 (segment (start 122.936 93.98) (end 121.666 95.25) (width 0.5) (layer F.Cu) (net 8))
 (segment (start 125.095 93.98) (end 122.936 93.98) (width 0.5) (layer F.Cu) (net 8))
 (via (at 153.67 99.06) (size 0.8) (drill 0.4) (layers F.Cu B.Cu) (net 9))
 (segment (start 134.874 101.6) (end 134.874 99.949) (width 0.5) (layer F.Cu) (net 9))
 (segment (start 155.194 99.06) (end 155.194 100.711) (width 0.5) (layer F.Cu) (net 9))
 (segment (start 134.874 99.695) (end 134.874 99.441) (width 0.5) (layer F.Cu) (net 9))
 (segment (start 125.095 88.9) (end 126.365 90.17) (width 0.5) (layer B.Cu) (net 9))
 (segment (start 126.365 90.17) (end 128.905 90.17) (width 0.5) (layer B.Cu) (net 9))
 (segment (start 128.905 90.17) (end 128.905 90.17) (width 0.5) (layer B.Cu) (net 9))
 (via (at 128.905 90.17) (size 0.8) (drill 0.4) (layers F.Cu B.Cu) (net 9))
 (segment (start 128.905 90.17) (end 130.175 90.17) (width 0.5) (layer F.Cu) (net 9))
 (segment (start 130.175 90.17) (end 132.08 92.075) (width 0.5) (layer F.Cu) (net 9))
 (segment (start 132.08 96.901) (end 132.08 92.075) (width 0.5) (layer F.Cu) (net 9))
 (segment (start 134.874 99.695) (end 133.477 98.298) (width 0.5) (layer F.Cu) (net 9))
 (segment (start 133.477 98.298) (end 132.08 96.901) (width 0.5) (layer F.Cu) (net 9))
 (via (at 132.969 97.79) (size 0.8) (drill 0.4) (layers F.Cu B.Cu) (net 9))
 (segment (start 153.67 99.06) (end 154.94 99.06) (width 0.5) (layer F.Cu) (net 9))
 (segment (start 133.985 97.79) (end 132.969 97.79) (width 0.5) (layer B.Cu) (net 9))
 (segment (start 152.4 97.79) (end 133.985 97.79) (width 0.5) (layer B.Cu) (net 9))
 (segment (start 153.67 99.06) (end 152.4 97.79) (width 0.5) (layer B.Cu) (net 9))
 (segment (start 117.856 88.9) (end 117.856 87.249) (width 0.5) (layer F.Cu) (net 10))
 (segment (start 118.745 88.9) (end 118.11 88.9) (width 0.5) (layer F.Cu) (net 10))
 (segment (start 118.745 88.9) (end 120.015 90.17) (width 0.5) (layer F.Cu) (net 10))
 (segment (start 120.015 90.17) (end 126.365 90.17) (width 0.5) (layer F.Cu) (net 10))
 (segment (start 126.365 90.17) (end 127.635 91.44) (width 0.5) (layer F.Cu) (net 10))
 (segment (start 127.635 96.52) (end 130.175 99.06) (width 0.5) (layer B.Cu) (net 11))
 (segment (start 130.175 99.06) (end 133.35 99.06) (width 0.5) (layer B.Cu) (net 11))
 (segment (start 133.35 99.06) (end 144.145 99.06) (width 0.5) (layer B.Cu) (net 11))
 (via (at 153.67 86.995) (size 0.8) (drill 0.4) (layers F.Cu B.Cu) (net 12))
 (segment (start 134.874 88.265) (end 134.874 86.614) (width 0.5) (layer F.Cu) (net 12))
 (segment (start 155.194 86.995) (end 155.194 88.646) (width 0.5) (layer F.Cu) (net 12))
 (segment (start 127.635 86.36) (end 133.35 86.36) (width 0.5) (layer F.Cu) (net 12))
 (segment (start 133.35 86.36) (end 134.62 86.36) (width 0.5) (layer F.Cu) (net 12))
 (via (at 133.35 86.36) (size 0.8) (drill 0.4) (layers F.Cu B.Cu) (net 12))
 (segment (start 153.67 86.995) (end 153.035 86.36) (width 0.5) (layer B.Cu) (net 12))
 (segment (start 133.35 86.36) (end 153.035 86.36) (width 0.5) (layer B.Cu) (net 12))
 (segment (start 153.67 86.995) (end 154.94 86.995) (width 0.5) (layer F.Cu) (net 12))
 (segment (start 117.856 92.71) (end 117.856 91.059) (width 0.5) (layer F.Cu) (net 13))
 (segment (start 117.856 90.805) (end 118.745 90.805) (width 0.5) (layer F.Cu) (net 13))
 (segment (start 118.745 90.805) (end 119.38 91.44) (width 0.5) (layer F.Cu) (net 13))
 (segment (start 119.38 91.44) (end 125.095 91.44) (width 0.5) (layer F.Cu) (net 13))
 (segment (start 172.8375 100.4475) (end 174.225 99.06) (width 0.5) (layer F.Cu) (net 14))
 (segment (start 163.3125 100.4475) (end 172.8375 100.4475) (width 0.5) (layer F.Cu) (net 14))
 (segment (start 161.525 102.235) (end 163.3125 100.4475) (width 0.5) (layer F.Cu) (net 14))
 (segment (start 139.76501 104.07499) (end 141.605 102.235) (width 0.5) (layer F.Cu) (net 14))
 (segment (start 132.64999 104.07499) (end 139.76501 104.07499) (width 0.5) (layer F.Cu) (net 14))
 (segment (start 128.905 100.33) (end 132.64999 104.07499) (width 0.5) (layer F.Cu) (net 14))
 (segment (start 126.365 100.33) (end 128.905 100.33) (width 0.5) (layer F.Cu) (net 14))
 (segment (start 141.605 102.235) (end 161.525 102.235) (width 0.5) (layer F.Cu) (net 14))
 (segment (start 125.095 99.06) (end 126.365 100.33) (width 0.5) (layer F.Cu) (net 14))
 (segment (start 115.824 90.805) (end 115.189 90.17) (width 0.5) (layer F.Cu) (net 24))
 (segment (start 115.189 90.17) (end 109.855 90.17) (width 0.5) (layer F.Cu) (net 24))
 (segment (start 109.855 90.17) (end 108.585 91.44) (width 0.5) (layer F.Cu) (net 24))
 (segment (start 108.585 91.44) (end 105.41 91.44) (width 0.5) (layer F.Cu) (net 24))
 (segment (start 107.95 88.9) (end 105.645 88.9) (width 0.5) (layer F.Cu) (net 23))
 (segment (start 109.855 86.995) (end 107.95 88.9) (width 0.5) (layer F.Cu) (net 23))
 (segment (start 115.824 86.995) (end 109.855 86.995) (width 0.5) (layer F.Cu) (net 23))
 (segment (start 115.824 100.965) (end 112.649 97.79) (width 0.5) (layer F.Cu) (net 25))
 (segment (start 112.649 97.79) (end 109.855 97.79) (width 0.5) (layer F.Cu) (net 25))
 (segment (start 109.855 97.79) (end 108.585 96.52) (width 0.5) (layer F.Cu) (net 25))
 (segment (start 108.585 96.52) (end 105.41 96.52) (width 0.5) (layer F.Cu) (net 25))
 (segment (start 115.824 97.155) (end 115.57 97.155) (width 0.5) (layer F.Cu) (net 26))
 (segment (start 115.57 97.155) (end 113.665 95.25) (width 0.5) (layer F.Cu) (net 26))
 (segment (start 113.665 95.25) (end 109.855 95.25) (width 0.5) (layer F.Cu) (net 26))
 (segment (start 109.855 95.25) (end 108.585 93.98) (width 0.5) (layer F.Cu) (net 26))
 (segment (start 108.585 93.98) (end 105.41 93.98) (width 0.5) (layer F.Cu) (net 26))
 (segment (start 115.824 88.9) (end 110.49 88.9) (width 0.5) (layer F.Cu) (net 19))
 (segment (start 115.824 92.71) (end 115.57 92.71) (width 0.5) (layer F.Cu) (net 20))
 (segment (start 115.57 92.71) (end 114.3 91.44) (width 0.5) (layer F.Cu) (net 20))
 (segment (start 114.3 91.44) (end 110.49 91.44) (width 0.5) (layer F.Cu) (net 20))
 (segment (start 115.824 95.25) (end 115.57 95.25) (width 0.5) (layer F.Cu) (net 22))
 (segment (start 115.57 95.25) (end 114.3 93.98) (width 0.5) (layer F.Cu) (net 22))
 (segment (start 114.3 93.98) (end 110.49 93.98) (width 0.5) (layer F.Cu) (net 22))
 (segment (start 115.824 99.06) (end 115.57 99.06) (width 0.5) (layer F.Cu) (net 21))
 (segment (start 115.57 99.06) (end 113.03 96.52) (width 0.5) (layer F.Cu) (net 21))
 (segment (start 113.03 96.52) (end 110.49 96.52) (width 0.5) (layer F.Cu) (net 21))
 (segment (start 136.906 92.71) (end 137.16 92.71) (width 0.5) (layer F.Cu) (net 16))
 (segment (start 137.16 92.71) (end 138.43 91.44) (width 0.5) (layer F.Cu) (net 16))
 (segment (start 138.43 91.44) (end 144.145 91.44) (width 0.5) (layer F.Cu) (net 16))
 (segment (start 136.906 88.265) (end 143.637 88.265) (width 0.5) (layer F.Cu) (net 15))
 (segment (start 143.637 88.265) (end 144.272 88.9) (width 0.5) (layer F.Cu) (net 15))
 (segment (start 136.906 99.695) (end 137.16 99.695) (width 0.5) (layer F.Cu) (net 17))
 (segment (start 137.16 99.695) (end 140.335 96.52) (width 0.5) (layer F.Cu) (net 17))
 (segment (start 140.335 96.52) (end 144.145 96.52) (width 0.5) (layer F.Cu) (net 17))
 (segment (start 136.906 86.36) (end 146.812 86.36) (width 0.5) (layer F.Cu) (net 35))
 (segment (start 146.812 86.36) (end 149.352 88.9) (width 0.5) (layer F.Cu) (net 35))
 (segment (start 136.906 95.25) (end 137.16 95.25) (width 0.5) (layer F.Cu) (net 18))
 (segment (start 137.16 95.25) (end 138.43 93.98) (width 0.5) (layer F.Cu) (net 18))
 (segment (start 138.43 93.98) (end 144.145 93.98) (width 0.5) (layer F.Cu) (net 18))
 (segment (start 136.906 97.155) (end 137.16 97.155) (width 0.5) (layer F.Cu) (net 38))
 (segment (start 137.16 97.155) (end 139.065 95.25) (width 0.5) (layer F.Cu) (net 38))
 (segment (start 139.065 95.25) (end 147.955 95.25) (width 0.5) (layer F.Cu) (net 38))
 (segment (start 147.955 95.25) (end 149.225 93.98) (width 0.5) (layer F.Cu) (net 38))
 (segment (start 136.906 90.805) (end 137.541 90.17) (width 0.5) (layer F.Cu) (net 36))
 (segment (start 137.541 90.17) (end 147.955 90.17) (width 0.5) (layer F.Cu) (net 36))
 (segment (start 147.955 90.17) (end 149.225 91.44) (width 0.5) (layer F.Cu) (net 36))
 (segment (start 136.906 101.6) (end 137.16 101.6) (width 0.5) (layer F.Cu) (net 37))
 (segment (start 140.850001 97.909999) (end 147.835001 97.909999) (width 0.5) (layer F.Cu) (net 37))
 (segment (start 137.16 101.6) (end 140.850001 97.909999) (width 0.5) (layer F.Cu) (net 37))
 (segment (start 147.835001 97.909999) (end 149.225 96.52) (width 0.5) (layer F.Cu) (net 37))
 (segment (start 159.766 88.9) (end 169.545 88.9) (width 0.5) (layer F.Cu) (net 31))
 (segment (start 157.226 88.9) (end 159.766 88.9) (width 0.5) (layer F.Cu) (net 31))
 (segment (start 157.226 92.71) (end 157.48 92.71) (width 0.5) (layer F.Cu) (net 32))
 (segment (start 160.02 92.71) (end 161.29 91.44) (width 0.5) (layer F.Cu) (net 32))
 (segment (start 161.29 91.44) (end 168.91 91.44) (width 0.5) (layer F.Cu) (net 32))
 (segment (start 160.02 92.71) (end 157.48 92.71) (width 0.5) (layer F.Cu) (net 32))
 (segment (start 157.226 95.25) (end 157.48 95.25) (width 0.5) (layer F.Cu) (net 34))
 (segment (start 160.02 95.25) (end 161.29 93.98) (width 0.5) (layer F.Cu) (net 34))
 (segment (start 161.29 93.98) (end 168.91 93.98) (width 0.5) (layer F.Cu) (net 34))
 (segment (start 157.226 95.25) (end 160.02 95.25) (width 0.5) (layer F.Cu) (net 34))
 (segment (start 157.226 99.06) (end 157.48 99.06) (width 0.5) (layer F.Cu) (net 33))
 (segment (start 160.02 99.06) (end 162.56 96.52) (width 0.5) (layer F.Cu) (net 33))
 (segment (start 162.56 96.52) (end 169.545 96.52) (width 0.5) (layer F.Cu) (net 33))
 (segment (start 160.02 99.06) (end 157.48 99.06) (width 0.5) (layer F.Cu) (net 33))
 (segment (start 159.766 86.995) (end 172.085 86.995) (width 0.5) (layer F.Cu) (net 27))
 (segment (start 172.32 86.995) (end 172.085 86.995) (width 0.5) (layer F.Cu) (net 27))
 (segment (start 174.225 88.9) (end 172.32 86.995) (width 0.5) (layer F.Cu) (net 27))
 (segment (start 159.766 86.995) (end 157.48 86.995) (width 0.5) (layer F.Cu) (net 27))
 (segment (start 157.226 97.155) (end 157.48 97.155) (width 0.5) (layer F.Cu) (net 30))
 (segment (start 160.02 97.155) (end 161.925 95.25) (width 0.5) (layer F.Cu) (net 30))
 (segment (start 161.925 95.25) (end 172.72 95.25) (width 0.5) (layer F.Cu) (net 30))
 (segment (start 172.72 95.25) (end 173.99 93.98) (width 0.5) (layer F.Cu) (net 30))
 (segment (start 157.226 97.155) (end 160.02 97.155) (width 0.5) (layer F.Cu) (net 30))
 (segment (start 160.02 90.805) (end 157.226 90.805) (width 0.5) (layer F.Cu) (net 28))
 (segment (start 160.935037 90.805) (end 160.02 90.805) (width 0.5) (layer F.Cu) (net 28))
 (segment (start 161.570037 90.17) (end 160.935037 90.805) (width 0.5) (layer F.Cu) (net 28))
 (segment (start 172.955 90.17) (end 161.570037 90.17) (width 0.5) (layer F.Cu) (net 28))
 (segment (start 174.225 91.44) (end 172.955 90.17) (width 0.5) (layer F.Cu) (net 28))
 (segment (start 157.226 100.965) (end 157.48 100.965) (width 0.5) (layer F.Cu) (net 29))
 (segment (start 160.02 100.965) (end 163.195 97.79) (width 0.5) (layer F.Cu) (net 29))
 (segment (start 163.195 97.79) (end 172.72 97.79) (width 0.5) (layer F.Cu) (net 29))
 (segment (start 172.72 97.79) (end 173.99 96.52) (width 0.5) (layer F.Cu) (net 29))
 (segment (start 157.226 100.965) (end 160.02 100.965) (width 0.5) (layer F.Cu) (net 29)))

